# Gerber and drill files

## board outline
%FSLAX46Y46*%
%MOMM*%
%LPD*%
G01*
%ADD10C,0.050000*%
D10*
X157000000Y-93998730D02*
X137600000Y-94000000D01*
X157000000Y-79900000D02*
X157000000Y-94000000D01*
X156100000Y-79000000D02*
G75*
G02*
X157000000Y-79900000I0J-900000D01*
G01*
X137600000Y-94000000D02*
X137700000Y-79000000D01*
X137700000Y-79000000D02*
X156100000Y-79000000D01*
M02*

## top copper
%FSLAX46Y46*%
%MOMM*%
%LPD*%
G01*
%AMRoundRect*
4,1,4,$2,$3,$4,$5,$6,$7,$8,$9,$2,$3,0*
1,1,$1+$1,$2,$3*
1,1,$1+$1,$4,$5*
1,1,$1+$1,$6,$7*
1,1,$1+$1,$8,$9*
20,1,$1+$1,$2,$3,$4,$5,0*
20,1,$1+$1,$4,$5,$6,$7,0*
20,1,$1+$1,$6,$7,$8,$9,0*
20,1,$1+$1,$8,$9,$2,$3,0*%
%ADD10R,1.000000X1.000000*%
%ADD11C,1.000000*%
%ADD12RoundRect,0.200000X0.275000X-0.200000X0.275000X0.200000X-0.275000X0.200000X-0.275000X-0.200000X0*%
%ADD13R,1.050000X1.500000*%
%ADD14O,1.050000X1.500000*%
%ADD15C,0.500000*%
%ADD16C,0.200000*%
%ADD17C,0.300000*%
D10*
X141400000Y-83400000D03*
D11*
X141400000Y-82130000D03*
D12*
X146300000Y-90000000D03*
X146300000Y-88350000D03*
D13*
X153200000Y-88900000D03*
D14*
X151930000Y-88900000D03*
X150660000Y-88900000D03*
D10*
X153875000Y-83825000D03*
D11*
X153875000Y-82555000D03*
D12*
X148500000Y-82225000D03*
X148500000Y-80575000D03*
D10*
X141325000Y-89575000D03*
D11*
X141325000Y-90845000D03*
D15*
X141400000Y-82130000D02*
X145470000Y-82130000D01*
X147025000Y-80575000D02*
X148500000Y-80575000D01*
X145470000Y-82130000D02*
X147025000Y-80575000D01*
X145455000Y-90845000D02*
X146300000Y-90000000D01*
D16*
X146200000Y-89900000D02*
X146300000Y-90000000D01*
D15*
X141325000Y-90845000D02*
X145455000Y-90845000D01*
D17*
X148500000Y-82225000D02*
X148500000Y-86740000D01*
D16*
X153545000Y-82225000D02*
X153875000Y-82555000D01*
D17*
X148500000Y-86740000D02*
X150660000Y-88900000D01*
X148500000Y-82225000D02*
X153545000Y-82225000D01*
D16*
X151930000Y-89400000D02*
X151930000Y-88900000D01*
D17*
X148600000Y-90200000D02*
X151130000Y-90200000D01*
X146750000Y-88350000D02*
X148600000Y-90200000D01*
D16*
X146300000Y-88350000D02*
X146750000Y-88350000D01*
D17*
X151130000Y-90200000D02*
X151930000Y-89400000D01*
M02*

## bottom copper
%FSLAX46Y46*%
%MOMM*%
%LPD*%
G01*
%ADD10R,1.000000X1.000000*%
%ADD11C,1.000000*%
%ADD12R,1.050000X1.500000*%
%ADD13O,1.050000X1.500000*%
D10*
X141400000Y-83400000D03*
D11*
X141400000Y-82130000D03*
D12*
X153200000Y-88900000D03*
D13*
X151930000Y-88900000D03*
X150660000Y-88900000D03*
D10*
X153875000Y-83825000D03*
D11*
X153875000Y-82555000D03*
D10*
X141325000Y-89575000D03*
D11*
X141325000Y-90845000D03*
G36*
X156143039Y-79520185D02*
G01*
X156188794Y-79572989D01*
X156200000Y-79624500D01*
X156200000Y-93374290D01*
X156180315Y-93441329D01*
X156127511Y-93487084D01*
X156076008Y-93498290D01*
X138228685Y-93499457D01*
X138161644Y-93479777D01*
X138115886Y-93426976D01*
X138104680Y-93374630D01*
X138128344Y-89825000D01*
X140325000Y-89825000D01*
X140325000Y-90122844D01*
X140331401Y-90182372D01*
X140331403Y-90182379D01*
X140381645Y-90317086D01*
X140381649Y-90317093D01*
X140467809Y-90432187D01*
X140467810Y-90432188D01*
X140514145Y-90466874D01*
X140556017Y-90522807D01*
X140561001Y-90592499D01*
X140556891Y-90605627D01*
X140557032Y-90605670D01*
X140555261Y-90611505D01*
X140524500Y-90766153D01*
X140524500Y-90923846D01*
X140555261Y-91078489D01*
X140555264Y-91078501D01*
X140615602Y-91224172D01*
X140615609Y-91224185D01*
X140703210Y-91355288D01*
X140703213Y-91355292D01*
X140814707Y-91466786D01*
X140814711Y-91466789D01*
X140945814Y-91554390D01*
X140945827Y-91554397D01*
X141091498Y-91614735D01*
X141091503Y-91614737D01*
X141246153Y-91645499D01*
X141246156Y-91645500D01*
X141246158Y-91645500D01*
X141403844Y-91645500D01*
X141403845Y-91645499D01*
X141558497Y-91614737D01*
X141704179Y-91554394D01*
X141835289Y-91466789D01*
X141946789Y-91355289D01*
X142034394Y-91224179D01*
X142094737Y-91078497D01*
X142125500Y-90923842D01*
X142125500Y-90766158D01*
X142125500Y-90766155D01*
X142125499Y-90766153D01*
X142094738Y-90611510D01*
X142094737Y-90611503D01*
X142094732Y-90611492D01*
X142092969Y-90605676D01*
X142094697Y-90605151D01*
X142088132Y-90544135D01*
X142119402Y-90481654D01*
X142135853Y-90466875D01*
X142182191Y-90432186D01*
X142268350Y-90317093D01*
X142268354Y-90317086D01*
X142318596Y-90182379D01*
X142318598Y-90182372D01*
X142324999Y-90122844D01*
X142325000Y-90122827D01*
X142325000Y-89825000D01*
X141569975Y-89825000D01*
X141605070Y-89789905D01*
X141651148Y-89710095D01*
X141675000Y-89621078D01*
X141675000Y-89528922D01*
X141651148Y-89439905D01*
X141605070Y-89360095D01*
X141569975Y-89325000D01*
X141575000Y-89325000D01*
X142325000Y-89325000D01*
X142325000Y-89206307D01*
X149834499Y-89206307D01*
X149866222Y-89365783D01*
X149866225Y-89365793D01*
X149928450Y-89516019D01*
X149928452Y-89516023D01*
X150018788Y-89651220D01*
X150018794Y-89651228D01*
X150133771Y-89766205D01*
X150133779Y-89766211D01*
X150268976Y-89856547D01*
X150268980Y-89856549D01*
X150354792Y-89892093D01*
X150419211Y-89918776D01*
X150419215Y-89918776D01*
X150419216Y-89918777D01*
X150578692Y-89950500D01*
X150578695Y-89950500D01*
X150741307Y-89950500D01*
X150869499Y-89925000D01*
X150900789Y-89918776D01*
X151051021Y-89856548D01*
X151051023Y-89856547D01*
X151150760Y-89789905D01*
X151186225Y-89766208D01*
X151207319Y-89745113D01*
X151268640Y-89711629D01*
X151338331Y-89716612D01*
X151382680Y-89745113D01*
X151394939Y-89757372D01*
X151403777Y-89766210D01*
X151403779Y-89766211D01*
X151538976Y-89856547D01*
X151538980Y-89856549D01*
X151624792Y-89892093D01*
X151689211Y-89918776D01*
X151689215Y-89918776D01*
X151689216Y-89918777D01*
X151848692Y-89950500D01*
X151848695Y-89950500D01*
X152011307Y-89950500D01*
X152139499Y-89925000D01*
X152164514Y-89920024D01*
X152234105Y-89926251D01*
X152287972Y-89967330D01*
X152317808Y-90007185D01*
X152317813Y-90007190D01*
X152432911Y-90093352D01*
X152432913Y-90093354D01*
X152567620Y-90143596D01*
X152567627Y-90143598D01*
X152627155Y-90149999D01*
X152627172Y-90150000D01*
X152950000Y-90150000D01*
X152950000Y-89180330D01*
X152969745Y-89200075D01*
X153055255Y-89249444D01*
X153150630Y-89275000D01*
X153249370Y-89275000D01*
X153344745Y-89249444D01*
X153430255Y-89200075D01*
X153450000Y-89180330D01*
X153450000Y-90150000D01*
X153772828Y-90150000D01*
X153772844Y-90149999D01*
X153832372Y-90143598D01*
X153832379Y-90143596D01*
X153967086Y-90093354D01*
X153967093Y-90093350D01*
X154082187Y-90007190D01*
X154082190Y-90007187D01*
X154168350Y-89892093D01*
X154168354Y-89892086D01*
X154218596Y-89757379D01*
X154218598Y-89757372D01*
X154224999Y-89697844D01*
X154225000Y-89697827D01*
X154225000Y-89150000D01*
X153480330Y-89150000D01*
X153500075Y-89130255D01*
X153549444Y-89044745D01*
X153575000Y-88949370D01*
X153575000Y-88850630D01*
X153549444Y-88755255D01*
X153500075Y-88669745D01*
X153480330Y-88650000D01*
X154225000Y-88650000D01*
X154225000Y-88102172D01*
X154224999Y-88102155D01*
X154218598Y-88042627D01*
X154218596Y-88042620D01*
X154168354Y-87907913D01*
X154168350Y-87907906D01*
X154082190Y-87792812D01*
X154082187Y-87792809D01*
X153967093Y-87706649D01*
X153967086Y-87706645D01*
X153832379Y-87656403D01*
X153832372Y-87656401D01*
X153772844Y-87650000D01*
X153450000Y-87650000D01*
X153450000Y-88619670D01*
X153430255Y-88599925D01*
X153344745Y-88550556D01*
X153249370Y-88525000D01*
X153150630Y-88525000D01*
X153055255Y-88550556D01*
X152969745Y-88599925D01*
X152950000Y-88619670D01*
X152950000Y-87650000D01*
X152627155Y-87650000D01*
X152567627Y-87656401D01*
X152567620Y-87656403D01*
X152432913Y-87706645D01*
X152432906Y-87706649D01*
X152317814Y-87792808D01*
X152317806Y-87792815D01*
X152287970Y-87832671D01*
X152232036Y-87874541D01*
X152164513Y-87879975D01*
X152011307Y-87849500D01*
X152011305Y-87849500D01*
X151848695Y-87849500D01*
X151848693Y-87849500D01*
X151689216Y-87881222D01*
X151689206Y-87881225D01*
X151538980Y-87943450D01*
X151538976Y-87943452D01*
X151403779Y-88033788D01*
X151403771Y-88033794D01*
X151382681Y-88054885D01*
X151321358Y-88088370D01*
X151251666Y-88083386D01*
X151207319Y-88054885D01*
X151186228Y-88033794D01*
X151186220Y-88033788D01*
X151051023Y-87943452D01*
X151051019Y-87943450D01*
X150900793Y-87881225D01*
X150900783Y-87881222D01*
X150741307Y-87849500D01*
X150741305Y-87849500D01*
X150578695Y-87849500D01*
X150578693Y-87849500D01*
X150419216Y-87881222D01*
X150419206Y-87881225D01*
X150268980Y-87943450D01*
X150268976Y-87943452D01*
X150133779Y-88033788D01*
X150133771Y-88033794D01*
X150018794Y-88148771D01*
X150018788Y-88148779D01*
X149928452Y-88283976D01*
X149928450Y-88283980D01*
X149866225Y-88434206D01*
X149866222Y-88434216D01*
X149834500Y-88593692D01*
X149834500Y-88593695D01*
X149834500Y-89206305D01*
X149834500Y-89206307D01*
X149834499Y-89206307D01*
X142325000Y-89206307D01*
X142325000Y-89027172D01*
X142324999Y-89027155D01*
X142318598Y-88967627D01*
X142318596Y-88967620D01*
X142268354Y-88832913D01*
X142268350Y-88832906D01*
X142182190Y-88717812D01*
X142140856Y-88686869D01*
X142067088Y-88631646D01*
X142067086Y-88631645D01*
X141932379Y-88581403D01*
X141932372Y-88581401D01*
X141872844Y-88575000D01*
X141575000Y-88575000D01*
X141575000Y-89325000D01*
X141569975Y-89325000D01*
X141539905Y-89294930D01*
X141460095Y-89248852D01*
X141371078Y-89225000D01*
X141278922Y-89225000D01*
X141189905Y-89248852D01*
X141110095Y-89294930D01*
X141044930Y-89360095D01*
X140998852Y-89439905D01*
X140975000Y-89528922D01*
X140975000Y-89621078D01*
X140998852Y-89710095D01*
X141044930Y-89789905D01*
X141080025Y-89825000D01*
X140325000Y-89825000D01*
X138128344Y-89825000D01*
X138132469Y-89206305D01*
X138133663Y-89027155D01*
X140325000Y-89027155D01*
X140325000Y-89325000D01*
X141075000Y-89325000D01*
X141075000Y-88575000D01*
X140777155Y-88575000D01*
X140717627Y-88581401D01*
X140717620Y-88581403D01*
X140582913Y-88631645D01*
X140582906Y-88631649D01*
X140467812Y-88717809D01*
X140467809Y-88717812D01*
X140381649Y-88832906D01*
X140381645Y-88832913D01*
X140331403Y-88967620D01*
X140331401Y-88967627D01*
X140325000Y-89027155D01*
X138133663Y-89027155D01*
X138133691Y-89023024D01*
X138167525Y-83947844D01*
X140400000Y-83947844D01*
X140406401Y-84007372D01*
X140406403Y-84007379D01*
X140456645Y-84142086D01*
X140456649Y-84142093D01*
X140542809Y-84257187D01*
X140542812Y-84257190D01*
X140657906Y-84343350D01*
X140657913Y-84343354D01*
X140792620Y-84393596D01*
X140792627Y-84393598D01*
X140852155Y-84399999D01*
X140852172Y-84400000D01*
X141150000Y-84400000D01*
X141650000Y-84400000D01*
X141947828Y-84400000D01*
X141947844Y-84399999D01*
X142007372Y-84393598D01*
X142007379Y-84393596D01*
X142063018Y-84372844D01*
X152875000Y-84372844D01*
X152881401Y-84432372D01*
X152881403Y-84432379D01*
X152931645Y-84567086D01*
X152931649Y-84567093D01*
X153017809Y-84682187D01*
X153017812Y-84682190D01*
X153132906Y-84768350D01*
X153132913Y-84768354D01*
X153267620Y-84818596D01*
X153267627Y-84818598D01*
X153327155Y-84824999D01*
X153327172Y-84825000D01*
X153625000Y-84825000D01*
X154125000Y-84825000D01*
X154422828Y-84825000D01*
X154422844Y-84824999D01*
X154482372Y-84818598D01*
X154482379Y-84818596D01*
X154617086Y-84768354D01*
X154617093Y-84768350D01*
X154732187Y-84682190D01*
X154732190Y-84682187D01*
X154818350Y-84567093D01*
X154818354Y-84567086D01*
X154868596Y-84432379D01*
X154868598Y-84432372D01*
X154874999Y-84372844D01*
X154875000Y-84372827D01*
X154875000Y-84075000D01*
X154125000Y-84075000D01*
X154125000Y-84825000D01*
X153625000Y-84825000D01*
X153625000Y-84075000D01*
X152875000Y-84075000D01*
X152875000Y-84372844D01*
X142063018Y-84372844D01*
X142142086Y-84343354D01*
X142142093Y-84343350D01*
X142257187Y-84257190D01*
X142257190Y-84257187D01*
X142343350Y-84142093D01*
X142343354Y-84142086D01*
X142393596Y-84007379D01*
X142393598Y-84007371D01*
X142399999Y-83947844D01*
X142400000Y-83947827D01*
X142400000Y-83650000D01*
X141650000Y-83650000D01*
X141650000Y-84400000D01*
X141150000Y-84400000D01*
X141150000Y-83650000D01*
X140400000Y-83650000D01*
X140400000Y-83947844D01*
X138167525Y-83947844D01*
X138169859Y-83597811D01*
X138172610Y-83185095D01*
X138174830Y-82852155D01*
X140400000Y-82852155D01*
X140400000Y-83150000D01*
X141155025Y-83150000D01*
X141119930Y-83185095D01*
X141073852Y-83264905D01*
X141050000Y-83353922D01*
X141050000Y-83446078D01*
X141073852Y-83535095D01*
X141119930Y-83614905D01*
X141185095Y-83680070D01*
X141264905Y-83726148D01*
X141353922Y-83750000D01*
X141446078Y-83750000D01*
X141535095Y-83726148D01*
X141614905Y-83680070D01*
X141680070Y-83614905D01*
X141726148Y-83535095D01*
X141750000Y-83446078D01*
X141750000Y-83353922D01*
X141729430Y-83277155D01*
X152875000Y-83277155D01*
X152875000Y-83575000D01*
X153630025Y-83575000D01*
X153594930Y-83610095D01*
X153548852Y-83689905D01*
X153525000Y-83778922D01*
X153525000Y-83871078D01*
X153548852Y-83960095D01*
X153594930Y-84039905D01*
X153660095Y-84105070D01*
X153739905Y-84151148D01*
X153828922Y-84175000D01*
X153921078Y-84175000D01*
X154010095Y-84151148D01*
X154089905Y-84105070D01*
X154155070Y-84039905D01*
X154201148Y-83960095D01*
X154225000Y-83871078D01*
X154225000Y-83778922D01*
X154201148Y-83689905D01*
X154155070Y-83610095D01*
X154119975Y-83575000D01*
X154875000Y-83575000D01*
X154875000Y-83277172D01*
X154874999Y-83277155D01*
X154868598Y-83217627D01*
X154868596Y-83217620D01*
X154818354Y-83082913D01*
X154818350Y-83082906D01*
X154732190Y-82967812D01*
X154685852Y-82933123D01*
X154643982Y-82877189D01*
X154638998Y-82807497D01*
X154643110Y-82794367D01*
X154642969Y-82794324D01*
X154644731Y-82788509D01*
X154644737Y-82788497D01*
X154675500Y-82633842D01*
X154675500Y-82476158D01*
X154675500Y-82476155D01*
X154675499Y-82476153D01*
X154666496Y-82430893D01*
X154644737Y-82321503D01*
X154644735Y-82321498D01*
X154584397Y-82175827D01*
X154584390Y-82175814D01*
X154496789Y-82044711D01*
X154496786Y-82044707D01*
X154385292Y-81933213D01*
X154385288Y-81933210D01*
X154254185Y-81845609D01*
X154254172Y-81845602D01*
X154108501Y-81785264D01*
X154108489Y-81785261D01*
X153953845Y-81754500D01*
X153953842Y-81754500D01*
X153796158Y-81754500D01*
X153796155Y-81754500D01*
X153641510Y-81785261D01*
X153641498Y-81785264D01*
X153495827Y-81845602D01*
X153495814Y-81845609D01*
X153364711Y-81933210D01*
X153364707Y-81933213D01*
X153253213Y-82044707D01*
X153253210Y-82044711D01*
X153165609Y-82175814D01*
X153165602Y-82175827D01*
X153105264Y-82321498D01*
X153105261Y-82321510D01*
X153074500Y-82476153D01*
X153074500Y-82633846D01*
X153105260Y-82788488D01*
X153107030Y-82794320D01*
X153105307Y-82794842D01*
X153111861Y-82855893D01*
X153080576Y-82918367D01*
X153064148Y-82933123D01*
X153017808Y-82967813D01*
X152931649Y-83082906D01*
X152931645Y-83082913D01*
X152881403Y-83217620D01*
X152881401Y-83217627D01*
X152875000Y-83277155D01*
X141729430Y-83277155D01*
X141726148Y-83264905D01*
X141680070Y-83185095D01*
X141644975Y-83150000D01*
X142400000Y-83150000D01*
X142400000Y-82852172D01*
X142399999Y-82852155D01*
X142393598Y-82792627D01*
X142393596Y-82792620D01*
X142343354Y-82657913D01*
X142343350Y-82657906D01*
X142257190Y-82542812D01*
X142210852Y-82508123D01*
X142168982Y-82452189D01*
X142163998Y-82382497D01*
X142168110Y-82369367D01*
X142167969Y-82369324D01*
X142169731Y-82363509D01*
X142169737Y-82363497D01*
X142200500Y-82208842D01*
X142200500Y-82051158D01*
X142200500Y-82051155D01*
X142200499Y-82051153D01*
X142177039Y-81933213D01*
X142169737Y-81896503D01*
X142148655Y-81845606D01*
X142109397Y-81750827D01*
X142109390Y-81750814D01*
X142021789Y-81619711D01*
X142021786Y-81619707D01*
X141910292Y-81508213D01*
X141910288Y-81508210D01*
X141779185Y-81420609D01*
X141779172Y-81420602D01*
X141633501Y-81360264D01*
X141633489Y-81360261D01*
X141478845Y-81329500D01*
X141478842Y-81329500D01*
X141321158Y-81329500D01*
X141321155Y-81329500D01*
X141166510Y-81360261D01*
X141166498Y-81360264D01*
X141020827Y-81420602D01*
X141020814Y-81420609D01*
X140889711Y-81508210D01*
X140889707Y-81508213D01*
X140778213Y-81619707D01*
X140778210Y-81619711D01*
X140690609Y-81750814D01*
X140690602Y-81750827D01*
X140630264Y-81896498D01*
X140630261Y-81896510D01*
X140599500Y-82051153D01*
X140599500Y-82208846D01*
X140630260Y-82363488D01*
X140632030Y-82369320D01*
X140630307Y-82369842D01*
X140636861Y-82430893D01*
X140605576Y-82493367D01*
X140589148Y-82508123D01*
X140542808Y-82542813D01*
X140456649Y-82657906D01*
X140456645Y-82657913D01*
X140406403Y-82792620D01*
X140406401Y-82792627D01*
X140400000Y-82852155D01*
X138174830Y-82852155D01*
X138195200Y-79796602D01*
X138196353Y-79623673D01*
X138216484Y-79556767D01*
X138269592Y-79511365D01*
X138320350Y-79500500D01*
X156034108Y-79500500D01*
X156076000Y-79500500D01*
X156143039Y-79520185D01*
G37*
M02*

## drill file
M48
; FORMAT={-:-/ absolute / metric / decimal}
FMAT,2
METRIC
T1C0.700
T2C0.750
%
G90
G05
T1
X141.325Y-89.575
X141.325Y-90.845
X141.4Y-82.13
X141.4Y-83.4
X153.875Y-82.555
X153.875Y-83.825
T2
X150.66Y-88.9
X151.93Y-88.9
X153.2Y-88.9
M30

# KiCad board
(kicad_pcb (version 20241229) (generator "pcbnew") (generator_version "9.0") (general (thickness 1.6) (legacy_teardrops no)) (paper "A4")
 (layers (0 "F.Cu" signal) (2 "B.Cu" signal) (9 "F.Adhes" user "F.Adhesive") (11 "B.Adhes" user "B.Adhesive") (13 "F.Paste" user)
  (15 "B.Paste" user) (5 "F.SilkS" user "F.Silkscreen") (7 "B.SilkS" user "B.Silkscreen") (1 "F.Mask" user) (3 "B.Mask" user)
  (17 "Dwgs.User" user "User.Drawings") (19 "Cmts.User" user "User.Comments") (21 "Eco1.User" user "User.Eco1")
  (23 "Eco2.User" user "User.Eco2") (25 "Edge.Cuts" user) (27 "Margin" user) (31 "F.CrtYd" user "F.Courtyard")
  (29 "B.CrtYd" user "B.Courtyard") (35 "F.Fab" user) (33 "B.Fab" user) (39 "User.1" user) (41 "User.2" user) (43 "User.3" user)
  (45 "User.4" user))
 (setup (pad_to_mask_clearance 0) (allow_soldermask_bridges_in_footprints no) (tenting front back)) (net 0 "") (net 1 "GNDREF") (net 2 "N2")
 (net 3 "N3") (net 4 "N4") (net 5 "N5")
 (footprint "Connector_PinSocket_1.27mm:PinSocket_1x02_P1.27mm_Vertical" (layer "F.Cu") (at 141.4 83.4 180)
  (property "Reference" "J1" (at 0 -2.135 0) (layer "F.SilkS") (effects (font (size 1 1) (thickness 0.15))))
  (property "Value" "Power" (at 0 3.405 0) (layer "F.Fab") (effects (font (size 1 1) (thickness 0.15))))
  (pad "1" thru_hole rect (at 0 0 180) (size 1 1) (drill 0.7) (layers "*.Cu" "*.Mask") (remove_unused_layers no) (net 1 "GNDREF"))
  (pad "2" thru_hole circle (at 0 1.27 180) (size 1 1) (drill 0.7) (layers "*.Cu" "*.Mask") (remove_unused_layers no) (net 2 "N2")))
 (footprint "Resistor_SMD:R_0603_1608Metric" (layer "F.Cu") (at 146.3 89.175 90)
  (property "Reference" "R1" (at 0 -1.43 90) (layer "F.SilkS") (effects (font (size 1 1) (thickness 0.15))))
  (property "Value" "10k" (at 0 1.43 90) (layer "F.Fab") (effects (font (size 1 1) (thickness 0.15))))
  (pad "1" smd roundrect (at -0.825 0 90) (size 0.8 0.95) (layers "F.Cu" "F.Mask" "F.Paste") (roundrect_rratio 0.25) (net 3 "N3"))
  (pad "2" smd roundrect (at 0.825 0 90) (size 0.8 0.95) (layers "F.Cu" "F.Mask" "F.Paste") (roundrect_rratio 0.25) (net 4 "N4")))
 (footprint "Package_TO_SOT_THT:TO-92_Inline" (layer "F.Cu") (at 153.2 88.9 180)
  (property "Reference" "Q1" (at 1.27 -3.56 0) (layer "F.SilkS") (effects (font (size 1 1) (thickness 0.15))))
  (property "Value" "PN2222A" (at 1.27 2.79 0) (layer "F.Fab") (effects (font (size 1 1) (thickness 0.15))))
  (pad "1" thru_hole rect (at 0 0 180) (size 1.05 1.5) (drill 0.75) (layers "*.Cu" "*.Mask") (remove_unused_layers no) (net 1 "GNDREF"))
  (pad "2" thru_hole oval (at 1.27 0 180) (size 1.05 1.5) (drill 0.75) (layers "*.Cu" "*.Mask") (remove_unused_layers no) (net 4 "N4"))
  (pad "3" thru_hole oval (at 2.54 0 180) (size 1.05 1.5) (drill 0.75) (layers "*.Cu" "*.Mask") (remove_unused_layers no) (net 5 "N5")))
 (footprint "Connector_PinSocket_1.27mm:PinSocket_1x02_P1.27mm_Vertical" (layer "F.Cu") (at 153.875 83.825 180)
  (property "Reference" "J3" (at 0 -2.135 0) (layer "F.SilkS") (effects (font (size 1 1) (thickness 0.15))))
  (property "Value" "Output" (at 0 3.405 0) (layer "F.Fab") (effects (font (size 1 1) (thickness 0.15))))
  (pad "1" thru_hole rect (at 0 0 180) (size 1 1) (drill 0.7) (layers "*.Cu" "*.Mask") (remove_unused_layers no) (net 1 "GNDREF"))
  (pad "2" thru_hole circle (at 0 1.27 180) (size 1 1) (drill 0.7) (layers "*.Cu" "*.Mask") (remove_unused_layers no) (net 5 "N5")))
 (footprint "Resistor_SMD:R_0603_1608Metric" (layer "F.Cu") (at 148.5 81.4 90)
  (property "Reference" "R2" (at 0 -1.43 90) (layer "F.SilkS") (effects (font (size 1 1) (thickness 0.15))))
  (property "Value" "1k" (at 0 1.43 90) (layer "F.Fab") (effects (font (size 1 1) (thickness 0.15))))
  (pad "1" smd roundrect (at -0.825 0 90) (size 0.8 0.95) (layers "F.Cu" "F.Mask" "F.Paste") (roundrect_rratio 0.25) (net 5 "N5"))
  (pad "2" smd roundrect (at 0.825 0 90) (size 0.8 0.95) (layers "F.Cu" "F.Mask" "F.Paste") (roundrect_rratio 0.25) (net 2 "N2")))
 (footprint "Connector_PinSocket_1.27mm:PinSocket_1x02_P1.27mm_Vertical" (layer "F.Cu") (at 141.325 89.575)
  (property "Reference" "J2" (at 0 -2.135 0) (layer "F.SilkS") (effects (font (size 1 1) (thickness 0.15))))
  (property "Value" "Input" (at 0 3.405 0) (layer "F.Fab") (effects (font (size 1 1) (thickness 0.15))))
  (pad "1" thru_hole rect (at 0 0) (size 1 1) (drill 0.7) (layers "*.Cu" "*.Mask") (remove_unused_layers no) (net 1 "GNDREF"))
  (pad "2" thru_hole circle (at 0 1.27) (size 1 1) (drill 0.7) (layers "*.Cu" "*.Mask") (remove_unused_layers no) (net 3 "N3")))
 (gr_line (start 157 93.99873) (end 137.6 94) (stroke (width 0.05) (type default)) (layer "Edge.Cuts"))
 (gr_line (start 157 79.9) (end 157 94) (stroke (width 0.05) (type default)) (layer "Edge.Cuts"))
 (gr_arc (start 156.1 79) (mid 156.736396 79.263604) (end 157 79.9) (stroke (width 0.05) (type default)) (layer "Edge.Cuts"))
 (gr_line (start 137.6 94) (end 137.7 79) (stroke (width 0.05) (type default)) (layer "Edge.Cuts"))
 (gr_line (start 137.7 79) (end 156.1 79) (stroke (width 0.05) (type default)) (layer "Edge.Cuts"))
 (segment (start 141.4 82.13) (end 145.47 82.13) (width 0.5) (layer "F.Cu") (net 2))
 (segment (start 147.025 80.575) (end 148.5 80.575) (width 0.5) (layer "F.Cu") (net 2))
 (segment (start 145.47 82.13) (end 147.025 80.575) (width 0.5) (layer "F.Cu") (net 2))
 (segment (start 145.455 90.845) (end 146.3 90) (width 0.5) (layer "F.Cu") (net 3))
 (segment (start 146.2 89.9) (end 146.3 90) (width 0.2) (layer "F.Cu") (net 3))
 (segment (start 141.325 90.845) (end 145.455 90.845) (width 0.5) (layer "F.Cu") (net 3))
 (segment (start 148.5 82.225) (end 148.5 86.74) (width 0.3) (layer "F.Cu") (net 5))
 (segment (start 153.545 82.225) (end 153.875 82.555) (width 0.2) (layer "F.Cu") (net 5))
 (segment (start 148.5 86.74) (end 150.66 88.9) (width 0.3) (layer "F.Cu") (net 5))
 (segment (start 148.5 82.225) (end 153.545 82.225) (width 0.3) (layer "F.Cu") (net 5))
 (segment (start 151.93 89.4) (end 151.93 88.9) (width 0.2) (layer "F.Cu") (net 4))
 (segment (start 148.6 90.2) (end 151.13 90.2) (width 0.3) (layer "F.Cu") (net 4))
 (segment (start 146.75 88.35) (end 148.6 90.2) (width 0.3) (layer "F.Cu") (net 4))
 (segment (start 146.3 88.35) (end 146.75 88.35) (width 0.2) (layer "F.Cu") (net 4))
 (segment (start 151.13 90.2) (end 151.93 89.4) (width 0.3) (layer "F.Cu") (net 4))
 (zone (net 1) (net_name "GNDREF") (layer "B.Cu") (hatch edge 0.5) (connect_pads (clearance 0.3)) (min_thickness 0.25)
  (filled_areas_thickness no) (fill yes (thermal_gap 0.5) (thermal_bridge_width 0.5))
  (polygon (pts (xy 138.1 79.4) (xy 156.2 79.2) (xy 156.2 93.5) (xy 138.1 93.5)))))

